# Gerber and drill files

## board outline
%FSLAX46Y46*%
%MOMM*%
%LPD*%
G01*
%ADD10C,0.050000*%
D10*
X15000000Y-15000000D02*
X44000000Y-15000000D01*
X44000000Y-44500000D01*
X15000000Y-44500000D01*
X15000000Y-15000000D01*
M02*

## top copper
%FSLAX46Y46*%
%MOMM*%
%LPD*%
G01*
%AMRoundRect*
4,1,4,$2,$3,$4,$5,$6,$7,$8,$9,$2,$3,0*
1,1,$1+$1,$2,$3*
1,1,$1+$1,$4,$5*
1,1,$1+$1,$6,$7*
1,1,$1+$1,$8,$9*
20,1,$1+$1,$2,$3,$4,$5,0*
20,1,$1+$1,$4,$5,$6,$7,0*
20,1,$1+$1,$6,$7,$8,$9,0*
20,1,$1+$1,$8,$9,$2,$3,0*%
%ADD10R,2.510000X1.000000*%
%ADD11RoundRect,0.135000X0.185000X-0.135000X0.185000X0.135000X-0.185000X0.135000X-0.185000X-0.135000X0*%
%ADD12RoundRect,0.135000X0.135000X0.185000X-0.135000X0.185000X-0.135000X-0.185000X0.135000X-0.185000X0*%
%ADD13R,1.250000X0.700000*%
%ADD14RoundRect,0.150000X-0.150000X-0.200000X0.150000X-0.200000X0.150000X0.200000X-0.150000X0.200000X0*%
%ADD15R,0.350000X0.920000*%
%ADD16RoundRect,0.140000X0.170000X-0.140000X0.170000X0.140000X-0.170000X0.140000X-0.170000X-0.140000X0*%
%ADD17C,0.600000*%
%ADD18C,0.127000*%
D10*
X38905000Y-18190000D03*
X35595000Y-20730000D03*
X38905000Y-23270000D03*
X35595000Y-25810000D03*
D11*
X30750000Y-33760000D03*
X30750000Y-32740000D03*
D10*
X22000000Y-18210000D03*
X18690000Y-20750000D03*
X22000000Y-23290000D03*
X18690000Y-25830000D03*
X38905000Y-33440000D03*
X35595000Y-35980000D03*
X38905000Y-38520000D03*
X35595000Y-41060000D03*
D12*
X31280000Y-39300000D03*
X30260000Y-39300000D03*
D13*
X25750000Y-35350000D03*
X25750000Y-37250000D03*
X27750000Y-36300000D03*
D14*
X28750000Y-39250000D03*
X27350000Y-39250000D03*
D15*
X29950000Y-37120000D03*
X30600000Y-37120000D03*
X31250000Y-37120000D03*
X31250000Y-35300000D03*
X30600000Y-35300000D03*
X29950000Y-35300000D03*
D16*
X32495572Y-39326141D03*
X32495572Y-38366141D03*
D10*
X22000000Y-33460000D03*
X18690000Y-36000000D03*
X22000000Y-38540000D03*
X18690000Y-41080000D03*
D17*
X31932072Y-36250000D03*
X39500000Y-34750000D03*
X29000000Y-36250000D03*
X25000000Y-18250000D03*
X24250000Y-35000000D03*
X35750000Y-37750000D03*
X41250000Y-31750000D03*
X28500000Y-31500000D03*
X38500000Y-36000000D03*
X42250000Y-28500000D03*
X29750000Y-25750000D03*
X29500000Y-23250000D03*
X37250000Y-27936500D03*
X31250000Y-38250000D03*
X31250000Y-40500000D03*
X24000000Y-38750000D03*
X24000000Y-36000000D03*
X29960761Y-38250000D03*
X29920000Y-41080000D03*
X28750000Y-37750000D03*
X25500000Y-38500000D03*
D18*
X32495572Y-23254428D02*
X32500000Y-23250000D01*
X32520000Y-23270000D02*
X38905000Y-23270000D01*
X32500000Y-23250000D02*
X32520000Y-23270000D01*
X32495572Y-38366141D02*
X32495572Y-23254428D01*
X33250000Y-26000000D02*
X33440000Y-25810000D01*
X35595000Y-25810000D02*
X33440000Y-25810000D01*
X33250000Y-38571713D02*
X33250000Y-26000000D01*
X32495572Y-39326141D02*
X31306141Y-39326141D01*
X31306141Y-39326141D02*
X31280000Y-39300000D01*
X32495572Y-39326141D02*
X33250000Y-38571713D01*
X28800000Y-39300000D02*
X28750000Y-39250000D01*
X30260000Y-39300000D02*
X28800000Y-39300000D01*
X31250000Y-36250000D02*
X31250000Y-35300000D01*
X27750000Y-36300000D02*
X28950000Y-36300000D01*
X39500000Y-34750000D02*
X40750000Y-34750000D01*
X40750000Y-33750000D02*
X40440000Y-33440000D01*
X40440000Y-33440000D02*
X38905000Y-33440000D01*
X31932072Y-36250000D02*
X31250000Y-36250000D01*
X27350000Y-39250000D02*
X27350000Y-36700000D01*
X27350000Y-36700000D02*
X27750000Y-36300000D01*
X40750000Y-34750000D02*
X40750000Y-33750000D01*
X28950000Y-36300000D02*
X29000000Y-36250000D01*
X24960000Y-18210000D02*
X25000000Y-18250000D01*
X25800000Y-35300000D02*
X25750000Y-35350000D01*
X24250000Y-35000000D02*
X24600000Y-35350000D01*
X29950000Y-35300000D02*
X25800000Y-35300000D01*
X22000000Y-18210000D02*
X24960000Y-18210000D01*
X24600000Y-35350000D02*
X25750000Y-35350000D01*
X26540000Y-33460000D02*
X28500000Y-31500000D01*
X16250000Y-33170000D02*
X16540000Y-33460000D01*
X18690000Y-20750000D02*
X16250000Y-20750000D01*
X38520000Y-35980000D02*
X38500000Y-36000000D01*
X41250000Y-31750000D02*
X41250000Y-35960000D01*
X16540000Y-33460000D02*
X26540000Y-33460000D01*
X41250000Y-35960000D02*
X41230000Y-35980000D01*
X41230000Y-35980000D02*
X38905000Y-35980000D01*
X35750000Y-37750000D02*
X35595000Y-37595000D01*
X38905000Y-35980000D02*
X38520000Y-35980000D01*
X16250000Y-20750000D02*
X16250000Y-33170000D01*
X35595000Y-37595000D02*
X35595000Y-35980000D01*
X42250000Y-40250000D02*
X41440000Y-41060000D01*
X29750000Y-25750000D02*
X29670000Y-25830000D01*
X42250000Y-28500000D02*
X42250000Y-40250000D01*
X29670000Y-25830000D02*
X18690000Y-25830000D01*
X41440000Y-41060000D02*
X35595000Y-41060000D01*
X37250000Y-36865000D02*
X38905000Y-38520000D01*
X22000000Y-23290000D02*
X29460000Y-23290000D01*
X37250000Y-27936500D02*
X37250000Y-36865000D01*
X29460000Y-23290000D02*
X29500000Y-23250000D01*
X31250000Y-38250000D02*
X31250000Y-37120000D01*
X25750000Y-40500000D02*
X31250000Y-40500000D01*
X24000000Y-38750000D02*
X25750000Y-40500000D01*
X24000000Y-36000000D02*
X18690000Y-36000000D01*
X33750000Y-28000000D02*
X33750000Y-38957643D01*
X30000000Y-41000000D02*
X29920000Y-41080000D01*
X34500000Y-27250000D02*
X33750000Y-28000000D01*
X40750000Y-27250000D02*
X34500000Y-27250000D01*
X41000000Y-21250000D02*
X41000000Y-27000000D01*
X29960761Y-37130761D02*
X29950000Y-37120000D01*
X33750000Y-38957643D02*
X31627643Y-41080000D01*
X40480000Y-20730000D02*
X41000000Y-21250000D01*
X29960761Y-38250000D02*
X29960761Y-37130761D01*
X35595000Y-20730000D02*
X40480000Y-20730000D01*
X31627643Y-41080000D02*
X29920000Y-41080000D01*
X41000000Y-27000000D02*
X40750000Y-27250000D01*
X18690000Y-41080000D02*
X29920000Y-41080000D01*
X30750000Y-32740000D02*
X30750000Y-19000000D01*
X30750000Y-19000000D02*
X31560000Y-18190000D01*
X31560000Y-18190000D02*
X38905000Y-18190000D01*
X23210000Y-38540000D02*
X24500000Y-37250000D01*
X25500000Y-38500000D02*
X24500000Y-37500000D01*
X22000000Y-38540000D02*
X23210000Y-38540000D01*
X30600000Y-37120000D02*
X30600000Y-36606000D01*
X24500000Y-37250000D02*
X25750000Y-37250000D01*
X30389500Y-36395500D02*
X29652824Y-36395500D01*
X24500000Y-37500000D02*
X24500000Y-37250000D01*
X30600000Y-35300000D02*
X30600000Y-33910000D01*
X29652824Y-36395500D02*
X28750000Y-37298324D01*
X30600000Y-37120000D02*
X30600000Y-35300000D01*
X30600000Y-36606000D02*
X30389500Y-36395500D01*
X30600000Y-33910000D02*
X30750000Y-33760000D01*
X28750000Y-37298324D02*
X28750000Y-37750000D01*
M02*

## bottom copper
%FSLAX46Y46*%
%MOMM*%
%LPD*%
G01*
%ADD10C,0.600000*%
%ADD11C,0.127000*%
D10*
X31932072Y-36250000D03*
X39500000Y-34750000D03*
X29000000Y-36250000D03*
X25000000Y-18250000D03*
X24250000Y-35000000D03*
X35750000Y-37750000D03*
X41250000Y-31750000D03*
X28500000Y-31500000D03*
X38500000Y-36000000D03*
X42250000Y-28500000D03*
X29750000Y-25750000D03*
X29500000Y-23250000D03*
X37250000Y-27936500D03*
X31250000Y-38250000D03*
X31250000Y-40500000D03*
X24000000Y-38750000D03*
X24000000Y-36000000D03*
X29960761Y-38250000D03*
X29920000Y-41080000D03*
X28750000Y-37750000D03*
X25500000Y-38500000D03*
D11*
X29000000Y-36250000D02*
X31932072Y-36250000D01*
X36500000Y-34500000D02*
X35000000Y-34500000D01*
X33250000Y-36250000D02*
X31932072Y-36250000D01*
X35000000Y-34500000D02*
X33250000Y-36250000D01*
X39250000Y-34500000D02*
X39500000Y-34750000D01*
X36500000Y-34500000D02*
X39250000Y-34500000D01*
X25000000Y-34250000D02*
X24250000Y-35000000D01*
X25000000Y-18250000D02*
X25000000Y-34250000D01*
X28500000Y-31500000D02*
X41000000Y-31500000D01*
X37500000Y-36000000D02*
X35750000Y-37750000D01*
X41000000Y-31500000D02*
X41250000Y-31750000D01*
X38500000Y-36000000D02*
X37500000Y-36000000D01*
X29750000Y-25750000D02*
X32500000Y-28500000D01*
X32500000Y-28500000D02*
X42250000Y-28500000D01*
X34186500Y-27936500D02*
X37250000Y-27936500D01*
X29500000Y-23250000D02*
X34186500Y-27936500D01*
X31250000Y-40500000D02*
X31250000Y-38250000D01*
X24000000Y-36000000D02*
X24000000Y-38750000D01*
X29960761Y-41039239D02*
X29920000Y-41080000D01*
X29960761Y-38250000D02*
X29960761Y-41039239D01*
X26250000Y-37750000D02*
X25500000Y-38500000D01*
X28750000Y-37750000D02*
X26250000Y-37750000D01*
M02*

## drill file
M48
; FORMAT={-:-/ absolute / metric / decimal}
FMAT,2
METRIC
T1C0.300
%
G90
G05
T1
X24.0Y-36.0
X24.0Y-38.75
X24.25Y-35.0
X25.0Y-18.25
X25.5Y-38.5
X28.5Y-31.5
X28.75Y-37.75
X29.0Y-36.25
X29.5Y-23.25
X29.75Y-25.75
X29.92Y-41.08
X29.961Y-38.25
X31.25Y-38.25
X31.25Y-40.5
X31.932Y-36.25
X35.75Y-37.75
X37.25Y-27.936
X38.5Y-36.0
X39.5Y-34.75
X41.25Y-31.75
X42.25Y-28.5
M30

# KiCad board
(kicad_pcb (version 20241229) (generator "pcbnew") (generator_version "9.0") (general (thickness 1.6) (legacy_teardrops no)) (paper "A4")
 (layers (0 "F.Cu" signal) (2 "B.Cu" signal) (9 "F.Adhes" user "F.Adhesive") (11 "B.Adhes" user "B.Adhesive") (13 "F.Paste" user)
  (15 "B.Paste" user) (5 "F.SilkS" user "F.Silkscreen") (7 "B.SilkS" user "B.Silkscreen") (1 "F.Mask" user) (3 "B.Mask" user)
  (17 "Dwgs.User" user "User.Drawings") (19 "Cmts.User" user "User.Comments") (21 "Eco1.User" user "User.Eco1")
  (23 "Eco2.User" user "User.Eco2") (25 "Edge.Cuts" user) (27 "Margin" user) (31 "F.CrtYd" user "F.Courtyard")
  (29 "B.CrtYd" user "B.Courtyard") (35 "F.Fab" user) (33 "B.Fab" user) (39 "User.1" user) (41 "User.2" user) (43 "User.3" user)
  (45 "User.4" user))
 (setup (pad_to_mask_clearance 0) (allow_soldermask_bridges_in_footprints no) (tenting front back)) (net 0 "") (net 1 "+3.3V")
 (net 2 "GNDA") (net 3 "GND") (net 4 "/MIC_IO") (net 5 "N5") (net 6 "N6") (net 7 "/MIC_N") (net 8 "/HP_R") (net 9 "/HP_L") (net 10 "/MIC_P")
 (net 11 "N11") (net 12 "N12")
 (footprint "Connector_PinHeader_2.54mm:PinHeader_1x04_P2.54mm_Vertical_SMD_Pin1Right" (layer "F.Cu") (at 37.25 22)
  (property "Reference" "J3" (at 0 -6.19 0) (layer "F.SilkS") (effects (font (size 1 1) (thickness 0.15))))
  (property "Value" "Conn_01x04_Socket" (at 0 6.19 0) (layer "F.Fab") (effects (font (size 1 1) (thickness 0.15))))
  (pad "1" smd rect (at 1.655 -3.81) (size 2.51 1) (layers "F.Cu" "F.Mask" "F.Paste") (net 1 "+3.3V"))
  (pad "2" smd rect (at -1.655 -1.27) (size 2.51 1) (layers "F.Cu" "F.Mask" "F.Paste") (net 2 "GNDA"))
  (pad "3" smd rect (at 1.655 1.27) (size 2.51 1) (layers "F.Cu" "F.Mask" "F.Paste") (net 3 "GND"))
  (pad "4" smd rect (at -1.655 3.81) (size 2.51 1) (layers "F.Cu" "F.Mask" "F.Paste") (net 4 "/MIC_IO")))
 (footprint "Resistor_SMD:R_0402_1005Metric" (layer "F.Cu") (at 30.75 33.25 90)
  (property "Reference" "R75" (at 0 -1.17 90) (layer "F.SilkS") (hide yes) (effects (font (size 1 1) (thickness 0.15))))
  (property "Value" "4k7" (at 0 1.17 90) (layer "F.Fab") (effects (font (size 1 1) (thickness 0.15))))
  (pad "1" smd roundrect (at -0.51 0 90) (size 0.54 0.64) (layers "F.Cu" "F.Mask" "F.Paste") (roundrect_rratio 0.25) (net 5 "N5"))
  (pad "2" smd roundrect (at 0.51 0 90) (size 0.54 0.64) (layers "F.Cu" "F.Mask" "F.Paste") (roundrect_rratio 0.25) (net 1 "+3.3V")))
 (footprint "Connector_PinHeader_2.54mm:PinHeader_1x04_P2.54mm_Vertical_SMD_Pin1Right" (layer "F.Cu") (at 20.345 22.02)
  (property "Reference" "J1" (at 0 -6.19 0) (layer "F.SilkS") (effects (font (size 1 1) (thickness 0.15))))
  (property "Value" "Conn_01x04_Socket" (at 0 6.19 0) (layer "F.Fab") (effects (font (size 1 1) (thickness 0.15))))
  (pad "1" smd rect (at 1.655 -3.81) (size 2.51 1) (layers "F.Cu" "F.Mask" "F.Paste") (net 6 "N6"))
  (pad "2" smd rect (at -1.655 -1.27) (size 2.51 1) (layers "F.Cu" "F.Mask" "F.Paste") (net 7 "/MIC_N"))
  (pad "3" smd rect (at 1.655 1.27) (size 2.51 1) (layers "F.Cu" "F.Mask" "F.Paste") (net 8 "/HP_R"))
  (pad "4" smd rect (at -1.655 3.81) (size 2.51 1) (layers "F.Cu" "F.Mask" "F.Paste") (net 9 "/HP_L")))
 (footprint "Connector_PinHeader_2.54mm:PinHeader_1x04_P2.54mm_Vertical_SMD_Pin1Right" (layer "F.Cu") (at 37.25 37.25)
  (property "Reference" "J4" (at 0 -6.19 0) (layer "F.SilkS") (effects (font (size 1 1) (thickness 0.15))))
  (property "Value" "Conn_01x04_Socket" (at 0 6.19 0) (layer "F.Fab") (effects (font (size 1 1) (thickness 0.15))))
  (pad "1" smd rect (at 1.655 -3.81) (size 2.51 1) (layers "F.Cu" "F.Mask" "F.Paste") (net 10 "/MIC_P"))
  (pad "2" smd rect (at -1.655 -1.27) (size 2.51 1) (layers "F.Cu" "F.Mask" "F.Paste") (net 7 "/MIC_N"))
  (pad "3" smd rect (at 1.655 1.27) (size 2.51 1) (layers "F.Cu" "F.Mask" "F.Paste") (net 8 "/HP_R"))
  (pad "4" smd rect (at -1.655 3.81) (size 2.51 1) (layers "F.Cu" "F.Mask" "F.Paste") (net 9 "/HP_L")))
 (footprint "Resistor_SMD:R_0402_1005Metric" (layer "F.Cu") (at 30.77 39.3 180)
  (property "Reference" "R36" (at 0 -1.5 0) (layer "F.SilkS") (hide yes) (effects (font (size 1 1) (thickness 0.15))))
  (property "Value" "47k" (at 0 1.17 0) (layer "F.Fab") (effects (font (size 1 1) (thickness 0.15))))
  (pad "1" smd roundrect (at -0.51 0 180) (size 0.54 0.64) (layers "F.Cu" "F.Mask" "F.Paste") (roundrect_rratio 0.25) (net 4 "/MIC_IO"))
  (pad "2" smd roundrect (at 0.51 0 180) (size 0.54 0.64) (layers "F.Cu" "F.Mask" "F.Paste") (roundrect_rratio 0.25) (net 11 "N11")))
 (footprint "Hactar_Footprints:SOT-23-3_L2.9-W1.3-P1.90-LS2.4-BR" (layer "F.Cu") (at 26.75 36.3 180)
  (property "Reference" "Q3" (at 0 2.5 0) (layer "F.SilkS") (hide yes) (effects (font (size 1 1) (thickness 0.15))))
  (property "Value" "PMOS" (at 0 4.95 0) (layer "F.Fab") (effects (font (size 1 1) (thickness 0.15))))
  (pad "1" smd rect (at 1 0.95 180) (size 1.25 0.7) (layers "F.Cu" "F.Mask" "F.Paste") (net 6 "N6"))
  (pad "2" smd rect (at 1 -0.95 180) (size 1.25 0.7) (layers "F.Cu" "F.Mask" "F.Paste") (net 5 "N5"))
  (pad "3" smd rect (at -1 0 180) (size 1.25 0.7) (layers "F.Cu" "F.Mask" "F.Paste") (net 10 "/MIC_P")))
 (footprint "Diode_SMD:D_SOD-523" (layer "F.Cu") (at 28.05 39.25 180)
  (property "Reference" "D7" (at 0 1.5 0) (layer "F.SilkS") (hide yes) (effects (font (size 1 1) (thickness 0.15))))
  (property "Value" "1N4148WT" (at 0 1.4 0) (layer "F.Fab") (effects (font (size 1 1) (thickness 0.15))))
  (pad "1" smd roundrect (at -0.7 0) (size 0.6 0.7) (layers "F.Cu" "F.Mask" "F.Paste") (roundrect_rratio 0.25) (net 11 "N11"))
  (pad "2" smd roundrect (at 0.7 0) (size 0.6 0.7) (layers "F.Cu" "F.Mask" "F.Paste") (roundrect_rratio 0.25) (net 10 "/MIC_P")))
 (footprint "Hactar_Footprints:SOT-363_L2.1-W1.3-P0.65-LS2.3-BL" (layer "F.Cu") (at 30.6 36.21)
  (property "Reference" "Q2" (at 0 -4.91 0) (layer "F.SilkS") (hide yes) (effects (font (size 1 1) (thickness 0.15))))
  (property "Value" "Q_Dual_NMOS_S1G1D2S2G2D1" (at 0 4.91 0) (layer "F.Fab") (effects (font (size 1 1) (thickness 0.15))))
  (pad "1" smd rect (at -0.65 0.91) (size 0.35 0.92) (layers "F.Cu" "F.Mask" "F.Paste") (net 2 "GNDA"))
  (pad "2" smd rect (at 0 0.91) (size 0.35 0.92) (layers "F.Cu" "F.Mask" "F.Paste") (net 5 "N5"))
  (pad "3" smd rect (at 0.65 0.91) (size 0.35 0.92) (layers "F.Cu" "F.Mask" "F.Paste") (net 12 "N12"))
  (pad "4" smd rect (at 0.65 -0.91) (size 0.35 0.92) (layers "F.Cu" "F.Mask" "F.Paste") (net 10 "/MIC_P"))
  (pad "5" smd rect (at 0 -0.91) (size 0.35 0.92) (layers "F.Cu" "F.Mask" "F.Paste") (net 5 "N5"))
  (pad "6" smd rect (at -0.65 -0.91) (size 0.35 0.92) (layers "F.Cu" "F.Mask" "F.Paste") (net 6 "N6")))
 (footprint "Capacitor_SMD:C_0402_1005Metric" (layer "F.Cu") (at 32.495572 38.846141 90)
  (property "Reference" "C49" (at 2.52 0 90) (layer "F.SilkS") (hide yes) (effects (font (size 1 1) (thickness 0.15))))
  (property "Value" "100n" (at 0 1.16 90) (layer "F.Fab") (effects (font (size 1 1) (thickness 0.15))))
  (pad "1" smd roundrect (at -0.48 0 90) (size 0.56 0.62) (layers "F.Cu" "F.Mask" "F.Paste") (roundrect_rratio 0.25) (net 4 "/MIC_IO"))
  (pad "2" smd roundrect (at 0.48 0 90) (size 0.56 0.62) (layers "F.Cu" "F.Mask" "F.Paste") (roundrect_rratio 0.25) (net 3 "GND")))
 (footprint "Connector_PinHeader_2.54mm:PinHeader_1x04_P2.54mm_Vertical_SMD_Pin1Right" (layer "F.Cu") (at 20.345 37.27)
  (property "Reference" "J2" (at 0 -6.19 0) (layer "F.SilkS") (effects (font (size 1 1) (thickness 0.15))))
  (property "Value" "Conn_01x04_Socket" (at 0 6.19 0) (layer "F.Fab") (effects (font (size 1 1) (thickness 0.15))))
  (pad "1" smd rect (at 1.655 -3.81) (size 2.51 1) (layers "F.Cu" "F.Mask" "F.Paste") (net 7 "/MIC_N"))
  (pad "2" smd rect (at -1.655 -1.27) (size 2.51 1) (layers "F.Cu" "F.Mask" "F.Paste") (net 12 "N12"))
  (pad "3" smd rect (at 1.655 1.27) (size 2.51 1) (layers "F.Cu" "F.Mask" "F.Paste") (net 5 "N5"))
  (pad "4" smd rect (at -1.655 3.81) (size 2.51 1) (layers "F.Cu" "F.Mask" "F.Paste") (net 2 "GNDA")))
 (gr_rect (start 15 15) (end 44 44.5) (stroke (width 0.05) (type solid)) (fill no) (layer "Edge.Cuts"))
 (segment (start 32.495572 23.254428) (end 32.5 23.25) (width 0.127) (layer "F.Cu") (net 3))
 (segment (start 32.52 23.27) (end 38.905 23.27) (width 0.127) (layer "F.Cu") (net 3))
 (segment (start 32.5 23.25) (end 32.52 23.27) (width 0.127) (layer "F.Cu") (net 3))
 (segment (start 32.495572 38.366141) (end 32.495572 23.254428) (width 0.127) (layer "F.Cu") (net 3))
 (segment (start 33.25 26) (end 33.44 25.81) (width 0.127) (layer "F.Cu") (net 4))
 (segment (start 35.595 25.81) (end 33.44 25.81) (width 0.127) (layer "F.Cu") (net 4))
 (segment (start 33.25 38.571713) (end 33.25 26) (width 0.127) (layer "F.Cu") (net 4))
 (segment (start 32.495572 39.326141) (end 31.306141 39.326141) (width 0.127) (layer "F.Cu") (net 4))
 (segment (start 31.306141 39.326141) (end 31.28 39.3) (width 0.127) (layer "F.Cu") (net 4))
 (segment (start 32.495572 39.326141) (end 33.25 38.571713) (width 0.127) (layer "F.Cu") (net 4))
 (segment (start 28.8 39.3) (end 28.75 39.25) (width 0.127) (layer "F.Cu") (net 11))
 (segment (start 30.26 39.3) (end 28.8 39.3) (width 0.127) (layer "F.Cu") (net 11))
 (segment (start 31.25 36.25) (end 31.25 35.3) (width 0.127) (layer "F.Cu") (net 10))
 (segment (start 27.75 36.3) (end 28.95 36.3) (width 0.127) (layer "F.Cu") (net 10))
 (segment (start 39.5 34.75) (end 40.75 34.75) (width 0.127) (layer "F.Cu") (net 10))
 (segment (start 40.75 33.75) (end 40.44 33.44) (width 0.127) (layer "F.Cu") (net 10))
 (segment (start 40.44 33.44) (end 38.905 33.44) (width 0.127) (layer "F.Cu") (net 10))
 (segment (start 31.932072 36.25) (end 31.25 36.25) (width 0.127) (layer "F.Cu") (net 10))
 (segment (start 27.35 39.25) (end 27.35 36.7) (width 0.127) (layer "F.Cu") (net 10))
 (segment (start 27.35 36.7) (end 27.75 36.3) (width 0.127) (layer "F.Cu") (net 10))
 (segment (start 40.75 34.75) (end 40.75 33.75) (width 0.127) (layer "F.Cu") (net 10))
 (segment (start 28.95 36.3) (end 29 36.25) (width 0.127) (layer "F.Cu") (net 10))
 (via (at 31.932072 36.25) (size 0.6) (drill 0.3) (layers "F.Cu" "B.Cu") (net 10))
 (via (at 39.5 34.75) (size 0.6) (drill 0.3) (layers "F.Cu" "B.Cu") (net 10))
 (via (at 29 36.25) (size 0.6) (drill 0.3) (layers "F.Cu" "B.Cu") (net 10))
 (segment (start 29 36.25) (end 31.932072 36.25) (width 0.127) (layer "B.Cu") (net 10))
 (segment (start 36.5 34.5) (end 35 34.5) (width 0.127) (layer "B.Cu") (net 10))
 (segment (start 33.25 36.25) (end 31.932072 36.25) (width 0.127) (layer "B.Cu") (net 10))
 (segment (start 35 34.5) (end 33.25 36.25) (width 0.127) (layer "B.Cu") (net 10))
 (segment (start 39.25 34.5) (end 39.5 34.75) (width 0.127) (layer "B.Cu") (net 10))
 (segment (start 36.5 34.5) (end 39.25 34.5) (width 0.127) (layer "B.Cu") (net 10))
 (segment (start 24.96 18.21) (end 25 18.25) (width 0.127) (layer "F.Cu") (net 6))
 (segment (start 25.8 35.3) (end 25.75 35.35) (width 0.127) (layer "F.Cu") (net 6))
 (segment (start 24.25 35) (end 24.6 35.35) (width 0.127) (layer "F.Cu") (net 6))
 (segment (start 29.95 35.3) (end 25.8 35.3) (width 0.127) (layer "F.Cu") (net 6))
 (segment (start 22 18.21) (end 24.96 18.21) (width 0.127) (layer "F.Cu") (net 6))
 (segment (start 24.6 35.35) (end 25.75 35.35) (width 0.127) (layer "F.Cu") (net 6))
 (via (at 25 18.25) (size 0.6) (drill 0.3) (layers "F.Cu" "B.Cu") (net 6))
 (via (at 24.25 35) (size 0.6) (drill 0.3) (layers "F.Cu" "B.Cu") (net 6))
 (segment (start 25 34.25) (end 24.25 35) (width 0.127) (layer "B.Cu") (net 6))
 (segment (start 25 18.25) (end 25 34.25) (width 0.127) (layer "B.Cu") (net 6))
 (segment (start 26.54 33.46) (end 28.5 31.5) (width 0.127) (layer "F.Cu") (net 7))
 (segment (start 16.25 33.17) (end 16.54 33.46) (width 0.127) (layer "F.Cu") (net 7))
 (segment (start 18.69 20.75) (end 16.25 20.75) (width 0.127) (layer "F.Cu") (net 7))
 (segment (start 38.52 35.98) (end 38.5 36) (width 0.127) (layer "F.Cu") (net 7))
 (segment (start 41.25 31.75) (end 41.25 35.96) (width 0.127) (layer "F.Cu") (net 7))
 (segment (start 16.54 33.46) (end 26.54 33.46) (width 0.127) (layer "F.Cu") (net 7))
 (segment (start 41.25 35.96) (end 41.23 35.98) (width 0.127) (layer "F.Cu") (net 7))
 (segment (start 41.23 35.98) (end 38.905 35.98) (width 0.127) (layer "F.Cu") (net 7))
 (segment (start 35.75 37.75) (end 35.595 37.595) (width 0.127) (layer "F.Cu") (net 7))
 (segment (start 38.905 35.98) (end 38.52 35.98) (width 0.127) (layer "F.Cu") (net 7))
 (segment (start 16.25 20.75) (end 16.25 33.17) (width 0.127) (layer "F.Cu") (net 7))
 (segment (start 35.595 37.595) (end 35.595 35.98) (width 0.127) (layer "F.Cu") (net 7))
 (via (at 35.75 37.75) (size 0.6) (drill 0.3) (layers "F.Cu" "B.Cu") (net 7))
 (via (at 41.25 31.75) (size 0.6) (drill 0.3) (layers "F.Cu" "B.Cu") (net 7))
 (via (at 28.5 31.5) (size 0.6) (drill 0.3) (layers "F.Cu" "B.Cu") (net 7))
 (via (at 38.5 36) (size 0.6) (drill 0.3) (layers "F.Cu" "B.Cu") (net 7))
 (segment (start 28.5 31.5) (end 41 31.5) (width 0.127) (layer "B.Cu") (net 7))
 (segment (start 37.5 36) (end 35.75 37.75) (width 0.127) (layer "B.Cu") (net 7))
 (segment (start 41 31.5) (end 41.25 31.75) (width 0.127) (layer "B.Cu") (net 7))
 (segment (start 38.5 36) (end 37.5 36) (width 0.127) (layer "B.Cu") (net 7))
 (segment (start 42.25 40.25) (end 41.44 41.06) (width 0.127) (layer "F.Cu") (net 9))
 (segment (start 29.75 25.75) (end 29.67 25.83) (width 0.127) (layer "F.Cu") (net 9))
 (segment (start 42.25 28.5) (end 42.25 40.25) (width 0.127) (layer "F.Cu") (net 9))
 (segment (start 29.67 25.83) (end 18.69 25.83) (width 0.127) (layer "F.Cu") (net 9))
 (segment (start 41.44 41.06) (end 35.595 41.06) (width 0.127) (layer "F.Cu") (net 9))
 (via (at 42.25 28.5) (size 0.6) (drill 0.3) (layers "F.Cu" "B.Cu") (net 9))
 (via (at 29.75 25.75) (size 0.6) (drill 0.3) (layers "F.Cu" "B.Cu") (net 9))
 (segment (start 29.75 25.75) (end 32.5 28.5) (width 0.127) (layer "B.Cu") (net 9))
 (segment (start 32.5 28.5) (end 42.25 28.5) (width 0.127) (layer "B.Cu") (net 9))
 (segment (start 37.25 36.865) (end 38.905 38.52) (width 0.127) (layer "F.Cu") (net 8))
 (segment (start 22 23.29) (end 29.46 23.29) (width 0.127) (layer "F.Cu") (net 8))
 (segment (start 37.25 27.9365) (end 37.25 36.865) (width 0.127) (layer "F.Cu") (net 8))
 (segment (start 29.46 23.29) (end 29.5 23.25) (width 0.127) (layer "F.Cu") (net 8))
 (via (at 29.5 23.25) (size 0.6) (drill 0.3) (layers "F.Cu" "B.Cu") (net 8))
 (via (at 37.25 27.9365) (size 0.6) (drill 0.3) (layers "F.Cu" "B.Cu") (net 8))
 (segment (start 34.1865 27.9365) (end 37.25 27.9365) (width 0.127) (layer "B.Cu") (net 8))
 (segment (start 29.5 23.25) (end 34.1865 27.9365) (width 0.127) (layer "B.Cu") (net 8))
 (segment (start 31.25 38.25) (end 31.25 37.12) (width 0.127) (layer "F.Cu") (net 12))
 (segment (start 25.75 40.5) (end 31.25 40.5) (width 0.127) (layer "F.Cu") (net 12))
 (segment (start 24 38.75) (end 25.75 40.5) (width 0.127) (layer "F.Cu") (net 12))
 (segment (start 24 36) (end 18.69 36) (width 0.127) (layer "F.Cu") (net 12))
 (via (at 31.25 38.25) (size 0.6) (drill 0.3) (layers "F.Cu" "B.Cu") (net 12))
 (via (at 31.25 40.5) (size 0.6) (drill 0.3) (layers "F.Cu" "B.Cu") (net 12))
 (via (at 24 38.75) (size 0.6) (drill 0.3) (layers "F.Cu" "B.Cu") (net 12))
 (via (at 24 36) (size 0.6) (drill 0.3) (layers "F.Cu" "B.Cu") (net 12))
 (segment (start 31.25 40.5) (end 31.25 38.25) (width 0.127) (layer "B.Cu") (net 12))
 (segment (start 24 36) (end 24 38.75) (width 0.127) (layer "B.Cu") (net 12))
 (segment (start 33.75 28) (end 33.75 38.957643) (width 0.127) (layer "F.Cu") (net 2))
 (segment (start 30 41) (end 29.92 41.08) (width 0.127) (layer "F.Cu") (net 2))
 (segment (start 34.5 27.25) (end 33.75 28) (width 0.127) (layer "F.Cu") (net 2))
 (segment (start 40.75 27.25) (end 34.5 27.25) (width 0.127) (layer "F.Cu") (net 2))
 (segment (start 41 21.25) (end 41 27) (width 0.127) (layer "F.Cu") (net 2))
 (segment (start 29.960761 37.130761) (end 29.95 37.12) (width 0.127) (layer "F.Cu") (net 2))
 (segment (start 33.75 38.957643) (end 31.627643 41.08) (width 0.127) (layer "F.Cu") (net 2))
 (segment (start 40.48 20.73) (end 41 21.25) (width 0.127) (layer "F.Cu") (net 2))
 (segment (start 29.960761 38.25) (end 29.960761 37.130761) (width 0.127) (layer "F.Cu") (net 2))
 (segment (start 35.595 20.73) (end 40.48 20.73) (width 0.127) (layer "F.Cu") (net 2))
 (segment (start 31.627643 41.08) (end 29.92 41.08) (width 0.127) (layer "F.Cu") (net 2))
 (segment (start 41 27) (end 40.75 27.25) (width 0.127) (layer "F.Cu") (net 2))
 (segment (start 18.69 41.08) (end 29.92 41.08) (width 0.127) (layer "F.Cu") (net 2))
 (via (at 29.960761 38.25) (size 0.6) (drill 0.3) (layers "F.Cu" "B.Cu") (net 2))
 (via (at 29.92 41.08) (size 0.6) (drill 0.3) (layers "F.Cu" "B.Cu") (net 2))
 (segment (start 29.960761 41.039239) (end 29.92 41.08) (width 0.127) (layer "B.Cu") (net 2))
 (segment (start 29.960761 38.25) (end 29.960761 41.039239) (width 0.127) (layer "B.Cu") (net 2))
 (segment (start 30.75 32.74) (end 30.75 19) (width 0.127) (layer "F.Cu") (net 1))
 (segment (start 30.75 19) (end 31.56 18.19) (width 0.127) (layer "F.Cu") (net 1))
 (segment (start 31.56 18.19) (end 38.905 18.19) (width 0.127) (layer "F.Cu") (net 1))
 (segment (start 23.21 38.54) (end 24.5 37.25) (width 0.127) (layer "F.Cu") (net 5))
 (segment (start 25.5 38.5) (end 24.5 37.5) (width 0.127) (layer "F.Cu") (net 5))
 (segment (start 22 38.54) (end 23.21 38.54) (width 0.127) (layer "F.Cu") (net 5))
 (segment (start 30.6 37.12) (end 30.6 36.606) (width 0.127) (layer "F.Cu") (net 5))
 (segment (start 24.5 37.25) (end 25.75 37.25) (width 0.127) (layer "F.Cu") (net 5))
 (segment (start 30.3895 36.3955) (end 29.652824 36.3955) (width 0.127) (layer "F.Cu") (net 5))
 (segment (start 24.5 37.5) (end 24.5 37.25) (width 0.127) (layer "F.Cu") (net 5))
 (segment (start 30.6 35.3) (end 30.6 33.91) (width 0.127) (layer "F.Cu") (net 5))
 (segment (start 29.652824 36.3955) (end 28.75 37.298324) (width 0.127) (layer "F.Cu") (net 5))
 (segment (start 30.6 37.12) (end 30.6 35.3) (width 0.127) (layer "F.Cu") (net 5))
 (segment (start 30.6 36.606) (end 30.3895 36.3955) (width 0.127) (layer "F.Cu") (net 5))
 (segment (start 30.6 33.91) (end 30.75 33.76) (width 0.127) (layer "F.Cu") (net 5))
 (segment (start 28.75 37.298324) (end 28.75 37.75) (width 0.127) (layer "F.Cu") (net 5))
 (via (at 28.75 37.75) (size 0.6) (drill 0.3) (layers "F.Cu" "B.Cu") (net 5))
 (via (at 25.5 38.5) (size 0.6) (drill 0.3) (layers "F.Cu" "B.Cu") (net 5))
 (segment (start 26.25 37.75) (end 25.5 38.5) (width 0.127) (layer "B.Cu") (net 5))
 (segment (start 28.75 37.75) (end 26.25 37.75) (width 0.127) (layer "B.Cu") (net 5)))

